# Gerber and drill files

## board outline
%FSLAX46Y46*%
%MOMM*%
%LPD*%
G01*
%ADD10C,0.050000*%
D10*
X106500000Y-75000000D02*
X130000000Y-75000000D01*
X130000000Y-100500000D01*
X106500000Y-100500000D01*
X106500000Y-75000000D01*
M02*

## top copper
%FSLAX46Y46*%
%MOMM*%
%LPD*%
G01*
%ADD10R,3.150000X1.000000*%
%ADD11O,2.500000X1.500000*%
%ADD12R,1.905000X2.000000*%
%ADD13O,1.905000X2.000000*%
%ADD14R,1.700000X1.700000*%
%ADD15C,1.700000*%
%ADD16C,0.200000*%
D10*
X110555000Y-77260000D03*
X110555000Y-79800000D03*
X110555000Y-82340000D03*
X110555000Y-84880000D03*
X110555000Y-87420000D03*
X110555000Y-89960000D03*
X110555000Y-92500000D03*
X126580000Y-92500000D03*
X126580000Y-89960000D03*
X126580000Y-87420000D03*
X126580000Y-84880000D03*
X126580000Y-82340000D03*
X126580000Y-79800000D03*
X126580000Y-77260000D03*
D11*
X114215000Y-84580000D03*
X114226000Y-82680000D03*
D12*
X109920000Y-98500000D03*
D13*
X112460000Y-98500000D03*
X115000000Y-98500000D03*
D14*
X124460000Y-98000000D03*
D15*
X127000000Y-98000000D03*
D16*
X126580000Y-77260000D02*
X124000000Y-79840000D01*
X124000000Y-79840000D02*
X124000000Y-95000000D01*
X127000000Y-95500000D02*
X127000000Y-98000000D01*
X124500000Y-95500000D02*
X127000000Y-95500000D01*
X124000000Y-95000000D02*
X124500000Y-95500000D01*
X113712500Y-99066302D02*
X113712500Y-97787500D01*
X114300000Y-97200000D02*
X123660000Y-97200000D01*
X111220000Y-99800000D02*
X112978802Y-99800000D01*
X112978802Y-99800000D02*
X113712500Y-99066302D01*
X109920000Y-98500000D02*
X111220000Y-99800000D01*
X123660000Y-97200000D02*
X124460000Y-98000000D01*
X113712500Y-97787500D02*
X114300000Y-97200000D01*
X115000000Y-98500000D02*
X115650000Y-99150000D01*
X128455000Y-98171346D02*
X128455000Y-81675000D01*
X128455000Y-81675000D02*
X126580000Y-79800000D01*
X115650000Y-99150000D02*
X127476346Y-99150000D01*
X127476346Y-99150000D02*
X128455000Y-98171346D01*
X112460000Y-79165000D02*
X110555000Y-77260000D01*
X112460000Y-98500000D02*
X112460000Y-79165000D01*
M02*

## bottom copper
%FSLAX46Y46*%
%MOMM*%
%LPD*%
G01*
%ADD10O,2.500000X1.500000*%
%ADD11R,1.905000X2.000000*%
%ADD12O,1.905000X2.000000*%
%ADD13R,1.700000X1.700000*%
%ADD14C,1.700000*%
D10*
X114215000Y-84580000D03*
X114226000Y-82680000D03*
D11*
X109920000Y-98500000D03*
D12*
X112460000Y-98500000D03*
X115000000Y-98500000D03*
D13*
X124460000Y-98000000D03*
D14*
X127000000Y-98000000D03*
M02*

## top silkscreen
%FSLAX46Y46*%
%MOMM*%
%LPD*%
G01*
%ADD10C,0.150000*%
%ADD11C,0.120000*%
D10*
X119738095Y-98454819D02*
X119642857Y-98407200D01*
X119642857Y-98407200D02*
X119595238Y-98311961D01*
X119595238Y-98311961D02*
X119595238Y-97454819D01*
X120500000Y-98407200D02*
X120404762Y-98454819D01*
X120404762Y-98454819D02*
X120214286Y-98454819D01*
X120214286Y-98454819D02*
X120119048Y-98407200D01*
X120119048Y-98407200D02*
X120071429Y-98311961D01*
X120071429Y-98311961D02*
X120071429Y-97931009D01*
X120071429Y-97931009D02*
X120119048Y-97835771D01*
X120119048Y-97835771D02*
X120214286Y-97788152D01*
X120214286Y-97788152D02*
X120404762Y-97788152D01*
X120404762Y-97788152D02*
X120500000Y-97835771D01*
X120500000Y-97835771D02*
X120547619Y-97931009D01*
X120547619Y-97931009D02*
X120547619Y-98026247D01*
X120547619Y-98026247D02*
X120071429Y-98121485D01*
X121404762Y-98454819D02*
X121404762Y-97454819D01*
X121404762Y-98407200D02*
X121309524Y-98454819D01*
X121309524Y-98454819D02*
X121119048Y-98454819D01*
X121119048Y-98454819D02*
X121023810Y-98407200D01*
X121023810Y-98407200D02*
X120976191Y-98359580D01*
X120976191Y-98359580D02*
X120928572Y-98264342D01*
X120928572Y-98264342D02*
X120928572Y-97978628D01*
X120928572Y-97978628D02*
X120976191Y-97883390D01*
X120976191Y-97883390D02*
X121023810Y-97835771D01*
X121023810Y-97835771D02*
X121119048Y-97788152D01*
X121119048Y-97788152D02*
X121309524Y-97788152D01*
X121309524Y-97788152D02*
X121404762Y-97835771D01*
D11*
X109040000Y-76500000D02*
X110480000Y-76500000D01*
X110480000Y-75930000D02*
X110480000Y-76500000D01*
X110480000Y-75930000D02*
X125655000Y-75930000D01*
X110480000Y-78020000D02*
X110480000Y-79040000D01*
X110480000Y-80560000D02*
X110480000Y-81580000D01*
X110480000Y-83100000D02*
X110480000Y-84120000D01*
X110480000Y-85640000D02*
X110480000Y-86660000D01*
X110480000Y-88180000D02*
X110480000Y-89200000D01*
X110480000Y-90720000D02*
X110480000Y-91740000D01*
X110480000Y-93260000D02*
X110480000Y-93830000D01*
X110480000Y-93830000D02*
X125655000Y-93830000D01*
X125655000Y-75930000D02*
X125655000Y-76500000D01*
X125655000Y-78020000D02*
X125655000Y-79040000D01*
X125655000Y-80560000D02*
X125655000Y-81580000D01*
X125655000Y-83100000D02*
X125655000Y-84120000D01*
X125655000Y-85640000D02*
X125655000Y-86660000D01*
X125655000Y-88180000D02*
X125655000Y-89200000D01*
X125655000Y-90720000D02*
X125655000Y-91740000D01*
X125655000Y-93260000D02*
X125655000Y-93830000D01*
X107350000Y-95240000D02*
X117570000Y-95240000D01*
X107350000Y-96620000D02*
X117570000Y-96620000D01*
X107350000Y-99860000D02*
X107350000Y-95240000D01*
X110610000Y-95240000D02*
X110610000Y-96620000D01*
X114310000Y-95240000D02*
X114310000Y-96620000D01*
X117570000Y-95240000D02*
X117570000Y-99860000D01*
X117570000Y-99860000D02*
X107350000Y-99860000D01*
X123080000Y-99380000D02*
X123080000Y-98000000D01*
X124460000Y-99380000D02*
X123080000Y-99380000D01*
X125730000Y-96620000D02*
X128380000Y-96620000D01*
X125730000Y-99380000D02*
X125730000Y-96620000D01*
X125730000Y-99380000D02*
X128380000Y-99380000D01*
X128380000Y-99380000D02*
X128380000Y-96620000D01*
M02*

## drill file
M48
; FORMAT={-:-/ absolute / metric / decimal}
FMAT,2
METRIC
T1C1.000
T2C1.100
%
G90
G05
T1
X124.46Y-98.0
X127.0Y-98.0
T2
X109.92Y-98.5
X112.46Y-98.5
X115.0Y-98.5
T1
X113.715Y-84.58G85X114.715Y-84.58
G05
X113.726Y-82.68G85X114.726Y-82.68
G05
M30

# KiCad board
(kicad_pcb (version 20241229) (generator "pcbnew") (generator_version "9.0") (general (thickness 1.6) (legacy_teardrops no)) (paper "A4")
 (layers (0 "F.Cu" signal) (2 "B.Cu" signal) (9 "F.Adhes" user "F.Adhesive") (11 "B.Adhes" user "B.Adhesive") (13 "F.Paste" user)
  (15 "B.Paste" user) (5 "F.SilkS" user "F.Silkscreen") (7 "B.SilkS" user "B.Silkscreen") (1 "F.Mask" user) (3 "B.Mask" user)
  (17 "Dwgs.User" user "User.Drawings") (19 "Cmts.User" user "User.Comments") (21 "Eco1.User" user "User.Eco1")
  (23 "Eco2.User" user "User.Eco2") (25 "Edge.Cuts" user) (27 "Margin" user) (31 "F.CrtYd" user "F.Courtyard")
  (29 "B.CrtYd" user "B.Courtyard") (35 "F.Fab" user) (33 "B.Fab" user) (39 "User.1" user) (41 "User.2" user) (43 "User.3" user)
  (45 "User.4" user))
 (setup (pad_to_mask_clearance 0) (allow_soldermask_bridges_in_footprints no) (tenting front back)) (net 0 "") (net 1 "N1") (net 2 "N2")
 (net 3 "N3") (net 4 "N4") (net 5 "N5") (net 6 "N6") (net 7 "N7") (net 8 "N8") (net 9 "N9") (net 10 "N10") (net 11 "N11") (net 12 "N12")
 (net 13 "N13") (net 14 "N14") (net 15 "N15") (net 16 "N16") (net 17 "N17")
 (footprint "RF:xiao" (layer "F.Cu") (at 119.155 86.68)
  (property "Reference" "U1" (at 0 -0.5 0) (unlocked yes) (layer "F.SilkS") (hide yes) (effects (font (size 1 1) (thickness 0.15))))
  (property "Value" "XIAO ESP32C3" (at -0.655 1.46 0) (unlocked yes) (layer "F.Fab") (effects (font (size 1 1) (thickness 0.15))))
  (fp_line (start -10.115 -10.18) (end -8.675 -10.18) (stroke (width 0.12) (type solid)) (layer "F.SilkS"))
  (fp_line (start -8.675 -10.75) (end -8.675 -10.18) (stroke (width 0.12) (type solid)) (layer "F.SilkS"))
  (fp_line (start -8.675 -10.75) (end 6.5 -10.75) (stroke (width 0.12) (type solid)) (layer "F.SilkS"))
  (fp_line (start -8.675 -8.66) (end -8.675 -7.64) (stroke (width 0.12) (type solid)) (layer "F.SilkS"))
  (fp_line (start -8.675 -6.12) (end -8.675 -5.1) (stroke (width 0.12) (type solid)) (layer "F.SilkS"))
  (fp_line (start -8.675 -3.58) (end -8.675 -2.56) (stroke (width 0.12) (type solid)) (layer "F.SilkS"))
  (fp_line (start -8.675 -1.04) (end -8.675 -0.02) (stroke (width 0.12) (type solid)) (layer "F.SilkS"))
  (fp_line (start -8.675 1.5) (end -8.675 2.52) (stroke (width 0.12) (type solid)) (layer "F.SilkS"))
  (fp_line (start -8.675 4.04) (end -8.675 5.06) (stroke (width 0.12) (type solid)) (layer "F.SilkS"))
  (fp_line (start -8.675 6.58) (end -8.675 7.15) (stroke (width 0.12) (type solid)) (layer "F.SilkS"))
  (fp_line (start -8.675 7.15) (end 6.5 7.15) (stroke (width 0.12) (type solid)) (layer "F.SilkS"))
  (fp_line (start 6.5 -10.75) (end 6.5 -10.18) (stroke (width 0.12) (type solid)) (layer "F.SilkS"))
  (fp_line (start 6.5 -8.66) (end 6.5 -7.64) (stroke (width 0.12) (type solid)) (layer "F.SilkS"))
  (fp_line (start 6.5 -6.12) (end 6.5 -5.1) (stroke (width 0.12) (type solid)) (layer "F.SilkS"))
  (fp_line (start 6.5 -3.58) (end 6.5 -2.56) (stroke (width 0.12) (type solid)) (layer "F.SilkS"))
  (fp_line (start 6.5 -1.04) (end 6.5 -0.02) (stroke (width 0.12) (type solid)) (layer "F.SilkS"))
  (fp_line (start 6.5 1.5) (end 6.5 2.52) (stroke (width 0.12) (type solid)) (layer "F.SilkS"))
  (fp_line (start 6.5 4.04) (end 6.5 5.06) (stroke (width 0.12) (type solid)) (layer "F.SilkS"))
  (fp_line (start 6.5 6.58) (end 6.5 7.15) (stroke (width 0.12) (type solid)) (layer "F.SilkS"))
  (pad "1" smd rect (at -8.6 -9.42) (size 3.15 1) (layers "F.Cu" "F.Mask" "F.Paste") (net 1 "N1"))
  (pad "2" smd rect (at -8.6 -6.88) (size 3.15 1) (layers "F.Cu" "F.Mask" "F.Paste") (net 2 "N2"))
  (pad "3" smd rect (at -8.6 -4.34) (size 3.15 1) (layers "F.Cu" "F.Mask" "F.Paste") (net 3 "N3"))
  (pad "4" smd rect (at -8.6 -1.8) (size 3.15 1) (layers "F.Cu" "F.Mask" "F.Paste") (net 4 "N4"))
  (pad "5" smd rect (at -8.6 0.74) (size 3.15 1) (layers "F.Cu" "F.Mask" "F.Paste") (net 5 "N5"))
  (pad "6" smd rect (at -8.6 3.28) (size 3.15 1) (layers "F.Cu" "F.Mask" "F.Paste") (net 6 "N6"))
  (pad "7" smd rect (at -8.6 5.82) (size 3.15 1) (layers "F.Cu" "F.Mask" "F.Paste") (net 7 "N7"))
  (pad "8" smd rect (at 7.425 5.82) (size 3.15 1) (layers "F.Cu" "F.Mask" "F.Paste") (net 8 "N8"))
  (pad "9" smd rect (at 7.425 3.28) (size 3.15 1) (layers "F.Cu" "F.Mask" "F.Paste") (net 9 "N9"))
  (pad "10" smd rect (at 7.425 0.74) (size 3.15 1) (layers "F.Cu" "F.Mask" "F.Paste") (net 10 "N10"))
  (pad "11" smd rect (at 7.425 -1.8) (size 3.15 1) (layers "F.Cu" "F.Mask" "F.Paste") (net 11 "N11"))
  (pad "12" smd rect (at 7.425 -4.34) (size 3.15 1) (layers "F.Cu" "F.Mask" "F.Paste") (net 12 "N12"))
  (pad "13" smd rect (at 7.425 -6.88) (size 3.15 1) (layers "F.Cu" "F.Mask" "F.Paste") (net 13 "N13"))
  (pad "14" smd rect (at 7.425 -9.42) (size 3.15 1) (layers "F.Cu" "F.Mask" "F.Paste") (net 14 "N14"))
  (pad "B+" thru_hole oval (at -4.94 -2.1) (size 2.5 1.5) (drill oval 2 1) (layers "*.Cu" "*.Mask") (remove_unused_layers no) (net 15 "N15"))
  (pad "B-" thru_hole oval (at -4.929 -4) (size 2.5 1.5) (drill oval 2 1) (layers "*.Cu" "*.Mask") (remove_unused_layers no) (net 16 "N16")))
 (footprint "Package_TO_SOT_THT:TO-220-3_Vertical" (layer "F.Cu") (at 109.92 98.5)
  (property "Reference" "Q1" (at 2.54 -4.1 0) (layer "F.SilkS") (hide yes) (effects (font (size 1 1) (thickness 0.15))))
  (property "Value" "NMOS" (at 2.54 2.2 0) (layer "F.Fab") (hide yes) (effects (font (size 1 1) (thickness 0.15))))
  (fp_line (start -2.57 -3.26) (end 7.65 -3.26) (stroke (width 0.12) (type solid)) (layer "F.SilkS"))
  (fp_line (start -2.57 -1.88) (end 7.65 -1.88) (stroke (width 0.12) (type solid)) (layer "F.SilkS"))
  (fp_line (start -2.57 1.36) (end -2.57 -3.26) (stroke (width 0.12) (type solid)) (layer "F.SilkS"))
  (fp_line (start 0.69 -3.26) (end 0.69 -1.88) (stroke (width 0.12) (type solid)) (layer "F.SilkS"))
  (fp_line (start 4.39 -3.26) (end 4.39 -1.88) (stroke (width 0.12) (type solid)) (layer "F.SilkS"))
  (fp_line (start 7.65 -3.26) (end 7.65 1.36) (stroke (width 0.12) (type solid)) (layer "F.SilkS"))
  (fp_line (start 7.65 1.36) (end -2.57 1.36) (stroke (width 0.12) (type solid)) (layer "F.SilkS"))
  (pad "1" thru_hole rect (at 0 0) (size 1.905 2) (drill 1.1) (layers "*.Cu" "*.Mask") (remove_unused_layers no) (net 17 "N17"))
  (pad "2" thru_hole oval (at 2.54 0) (size 1.905 2) (drill 1.1) (layers "*.Cu" "*.Mask") (remove_unused_layers no) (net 1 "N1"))
  (pad "3" thru_hole oval (at 5.08 0) (size 1.905 2) (drill 1.1) (layers "*.Cu" "*.Mask") (remove_unused_layers no) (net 13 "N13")))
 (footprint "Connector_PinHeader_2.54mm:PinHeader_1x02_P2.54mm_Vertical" (layer "F.Cu") (at 124.46 98 90)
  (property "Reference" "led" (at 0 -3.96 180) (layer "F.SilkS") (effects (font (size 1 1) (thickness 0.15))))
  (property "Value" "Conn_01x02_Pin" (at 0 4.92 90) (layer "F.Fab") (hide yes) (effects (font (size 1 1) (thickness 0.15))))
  (fp_line (start -1.38 -1.38) (end 0 -1.38) (stroke (width 0.12) (type solid)) (layer "F.SilkS"))
  (fp_line (start -1.38 0) (end -1.38 -1.38) (stroke (width 0.12) (type solid)) (layer "F.SilkS"))
  (fp_line (start 1.38 1.27) (end 1.38 3.92) (stroke (width 0.12) (type solid)) (layer "F.SilkS"))
  (fp_line (start -1.38 1.27) (end 1.38 1.27) (stroke (width 0.12) (type solid)) (layer "F.SilkS"))
  (fp_line (start -1.38 1.27) (end -1.38 3.92) (stroke (width 0.12) (type solid)) (layer "F.SilkS"))
  (fp_line (start -1.38 3.92) (end 1.38 3.92) (stroke (width 0.12) (type solid)) (layer "F.SilkS"))
  (pad "1" thru_hole rect (at 0 0 90) (size 1.7 1.7) (drill 1) (layers "*.Cu" "*.Mask") (remove_unused_layers no) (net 17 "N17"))
  (pad "2" thru_hole circle (at 0 2.54 90) (size 1.7 1.7) (drill 1) (layers "*.Cu" "*.Mask") (remove_unused_layers no) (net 14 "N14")))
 (gr_rect (start 106.5 75) (end 130 100.5) (stroke (width 0.05) (type default)) (fill no) (layer "Edge.Cuts"))
 (segment (start 126.58 77.26) (end 124 79.84) (width 0.2) (layer "F.Cu") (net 14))
 (segment (start 124 79.84) (end 124 95) (width 0.2) (layer "F.Cu") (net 14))
 (segment (start 127 95.5) (end 127 98) (width 0.2) (layer "F.Cu") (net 14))
 (segment (start 124.5 95.5) (end 127 95.5) (width 0.2) (layer "F.Cu") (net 14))
 (segment (start 124 95) (end 124.5 95.5) (width 0.2) (layer "F.Cu") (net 14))
 (segment (start 113.7125 99.066302) (end 113.7125 97.7875) (width 0.2) (layer "F.Cu") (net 17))
 (segment (start 114.3 97.2) (end 123.66 97.2) (width 0.2) (layer "F.Cu") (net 17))
 (segment (start 111.22 99.8) (end 112.978802 99.8) (width 0.2) (layer "F.Cu") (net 17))
 (segment (start 112.978802 99.8) (end 113.7125 99.066302) (width 0.2) (layer "F.Cu") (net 17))
 (segment (start 109.92 98.5) (end 111.22 99.8) (width 0.2) (layer "F.Cu") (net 17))
 (segment (start 123.66 97.2) (end 124.46 98) (width 0.2) (layer "F.Cu") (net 17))
 (segment (start 113.7125 97.7875) (end 114.3 97.2) (width 0.2) (layer "F.Cu") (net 17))
 (segment (start 115 98.5) (end 115.65 99.15) (width 0.2) (layer "F.Cu") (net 13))
 (segment (start 128.455 98.171346) (end 128.455 81.675) (width 0.2) (layer "F.Cu") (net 13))
 (segment (start 128.455 81.675) (end 126.58 79.8) (width 0.2) (layer "F.Cu") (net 13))
 (segment (start 115.65 99.15) (end 127.476346 99.15) (width 0.2) (layer "F.Cu") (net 13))
 (segment (start 127.476346 99.15) (end 128.455 98.171346) (width 0.2) (layer "F.Cu") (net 13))
 (segment (start 112.46 79.165) (end 110.555 77.26) (width 0.2) (layer "F.Cu") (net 1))
 (segment (start 112.46 98.5) (end 112.46 79.165) (width 0.2) (layer "F.Cu") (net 1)))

